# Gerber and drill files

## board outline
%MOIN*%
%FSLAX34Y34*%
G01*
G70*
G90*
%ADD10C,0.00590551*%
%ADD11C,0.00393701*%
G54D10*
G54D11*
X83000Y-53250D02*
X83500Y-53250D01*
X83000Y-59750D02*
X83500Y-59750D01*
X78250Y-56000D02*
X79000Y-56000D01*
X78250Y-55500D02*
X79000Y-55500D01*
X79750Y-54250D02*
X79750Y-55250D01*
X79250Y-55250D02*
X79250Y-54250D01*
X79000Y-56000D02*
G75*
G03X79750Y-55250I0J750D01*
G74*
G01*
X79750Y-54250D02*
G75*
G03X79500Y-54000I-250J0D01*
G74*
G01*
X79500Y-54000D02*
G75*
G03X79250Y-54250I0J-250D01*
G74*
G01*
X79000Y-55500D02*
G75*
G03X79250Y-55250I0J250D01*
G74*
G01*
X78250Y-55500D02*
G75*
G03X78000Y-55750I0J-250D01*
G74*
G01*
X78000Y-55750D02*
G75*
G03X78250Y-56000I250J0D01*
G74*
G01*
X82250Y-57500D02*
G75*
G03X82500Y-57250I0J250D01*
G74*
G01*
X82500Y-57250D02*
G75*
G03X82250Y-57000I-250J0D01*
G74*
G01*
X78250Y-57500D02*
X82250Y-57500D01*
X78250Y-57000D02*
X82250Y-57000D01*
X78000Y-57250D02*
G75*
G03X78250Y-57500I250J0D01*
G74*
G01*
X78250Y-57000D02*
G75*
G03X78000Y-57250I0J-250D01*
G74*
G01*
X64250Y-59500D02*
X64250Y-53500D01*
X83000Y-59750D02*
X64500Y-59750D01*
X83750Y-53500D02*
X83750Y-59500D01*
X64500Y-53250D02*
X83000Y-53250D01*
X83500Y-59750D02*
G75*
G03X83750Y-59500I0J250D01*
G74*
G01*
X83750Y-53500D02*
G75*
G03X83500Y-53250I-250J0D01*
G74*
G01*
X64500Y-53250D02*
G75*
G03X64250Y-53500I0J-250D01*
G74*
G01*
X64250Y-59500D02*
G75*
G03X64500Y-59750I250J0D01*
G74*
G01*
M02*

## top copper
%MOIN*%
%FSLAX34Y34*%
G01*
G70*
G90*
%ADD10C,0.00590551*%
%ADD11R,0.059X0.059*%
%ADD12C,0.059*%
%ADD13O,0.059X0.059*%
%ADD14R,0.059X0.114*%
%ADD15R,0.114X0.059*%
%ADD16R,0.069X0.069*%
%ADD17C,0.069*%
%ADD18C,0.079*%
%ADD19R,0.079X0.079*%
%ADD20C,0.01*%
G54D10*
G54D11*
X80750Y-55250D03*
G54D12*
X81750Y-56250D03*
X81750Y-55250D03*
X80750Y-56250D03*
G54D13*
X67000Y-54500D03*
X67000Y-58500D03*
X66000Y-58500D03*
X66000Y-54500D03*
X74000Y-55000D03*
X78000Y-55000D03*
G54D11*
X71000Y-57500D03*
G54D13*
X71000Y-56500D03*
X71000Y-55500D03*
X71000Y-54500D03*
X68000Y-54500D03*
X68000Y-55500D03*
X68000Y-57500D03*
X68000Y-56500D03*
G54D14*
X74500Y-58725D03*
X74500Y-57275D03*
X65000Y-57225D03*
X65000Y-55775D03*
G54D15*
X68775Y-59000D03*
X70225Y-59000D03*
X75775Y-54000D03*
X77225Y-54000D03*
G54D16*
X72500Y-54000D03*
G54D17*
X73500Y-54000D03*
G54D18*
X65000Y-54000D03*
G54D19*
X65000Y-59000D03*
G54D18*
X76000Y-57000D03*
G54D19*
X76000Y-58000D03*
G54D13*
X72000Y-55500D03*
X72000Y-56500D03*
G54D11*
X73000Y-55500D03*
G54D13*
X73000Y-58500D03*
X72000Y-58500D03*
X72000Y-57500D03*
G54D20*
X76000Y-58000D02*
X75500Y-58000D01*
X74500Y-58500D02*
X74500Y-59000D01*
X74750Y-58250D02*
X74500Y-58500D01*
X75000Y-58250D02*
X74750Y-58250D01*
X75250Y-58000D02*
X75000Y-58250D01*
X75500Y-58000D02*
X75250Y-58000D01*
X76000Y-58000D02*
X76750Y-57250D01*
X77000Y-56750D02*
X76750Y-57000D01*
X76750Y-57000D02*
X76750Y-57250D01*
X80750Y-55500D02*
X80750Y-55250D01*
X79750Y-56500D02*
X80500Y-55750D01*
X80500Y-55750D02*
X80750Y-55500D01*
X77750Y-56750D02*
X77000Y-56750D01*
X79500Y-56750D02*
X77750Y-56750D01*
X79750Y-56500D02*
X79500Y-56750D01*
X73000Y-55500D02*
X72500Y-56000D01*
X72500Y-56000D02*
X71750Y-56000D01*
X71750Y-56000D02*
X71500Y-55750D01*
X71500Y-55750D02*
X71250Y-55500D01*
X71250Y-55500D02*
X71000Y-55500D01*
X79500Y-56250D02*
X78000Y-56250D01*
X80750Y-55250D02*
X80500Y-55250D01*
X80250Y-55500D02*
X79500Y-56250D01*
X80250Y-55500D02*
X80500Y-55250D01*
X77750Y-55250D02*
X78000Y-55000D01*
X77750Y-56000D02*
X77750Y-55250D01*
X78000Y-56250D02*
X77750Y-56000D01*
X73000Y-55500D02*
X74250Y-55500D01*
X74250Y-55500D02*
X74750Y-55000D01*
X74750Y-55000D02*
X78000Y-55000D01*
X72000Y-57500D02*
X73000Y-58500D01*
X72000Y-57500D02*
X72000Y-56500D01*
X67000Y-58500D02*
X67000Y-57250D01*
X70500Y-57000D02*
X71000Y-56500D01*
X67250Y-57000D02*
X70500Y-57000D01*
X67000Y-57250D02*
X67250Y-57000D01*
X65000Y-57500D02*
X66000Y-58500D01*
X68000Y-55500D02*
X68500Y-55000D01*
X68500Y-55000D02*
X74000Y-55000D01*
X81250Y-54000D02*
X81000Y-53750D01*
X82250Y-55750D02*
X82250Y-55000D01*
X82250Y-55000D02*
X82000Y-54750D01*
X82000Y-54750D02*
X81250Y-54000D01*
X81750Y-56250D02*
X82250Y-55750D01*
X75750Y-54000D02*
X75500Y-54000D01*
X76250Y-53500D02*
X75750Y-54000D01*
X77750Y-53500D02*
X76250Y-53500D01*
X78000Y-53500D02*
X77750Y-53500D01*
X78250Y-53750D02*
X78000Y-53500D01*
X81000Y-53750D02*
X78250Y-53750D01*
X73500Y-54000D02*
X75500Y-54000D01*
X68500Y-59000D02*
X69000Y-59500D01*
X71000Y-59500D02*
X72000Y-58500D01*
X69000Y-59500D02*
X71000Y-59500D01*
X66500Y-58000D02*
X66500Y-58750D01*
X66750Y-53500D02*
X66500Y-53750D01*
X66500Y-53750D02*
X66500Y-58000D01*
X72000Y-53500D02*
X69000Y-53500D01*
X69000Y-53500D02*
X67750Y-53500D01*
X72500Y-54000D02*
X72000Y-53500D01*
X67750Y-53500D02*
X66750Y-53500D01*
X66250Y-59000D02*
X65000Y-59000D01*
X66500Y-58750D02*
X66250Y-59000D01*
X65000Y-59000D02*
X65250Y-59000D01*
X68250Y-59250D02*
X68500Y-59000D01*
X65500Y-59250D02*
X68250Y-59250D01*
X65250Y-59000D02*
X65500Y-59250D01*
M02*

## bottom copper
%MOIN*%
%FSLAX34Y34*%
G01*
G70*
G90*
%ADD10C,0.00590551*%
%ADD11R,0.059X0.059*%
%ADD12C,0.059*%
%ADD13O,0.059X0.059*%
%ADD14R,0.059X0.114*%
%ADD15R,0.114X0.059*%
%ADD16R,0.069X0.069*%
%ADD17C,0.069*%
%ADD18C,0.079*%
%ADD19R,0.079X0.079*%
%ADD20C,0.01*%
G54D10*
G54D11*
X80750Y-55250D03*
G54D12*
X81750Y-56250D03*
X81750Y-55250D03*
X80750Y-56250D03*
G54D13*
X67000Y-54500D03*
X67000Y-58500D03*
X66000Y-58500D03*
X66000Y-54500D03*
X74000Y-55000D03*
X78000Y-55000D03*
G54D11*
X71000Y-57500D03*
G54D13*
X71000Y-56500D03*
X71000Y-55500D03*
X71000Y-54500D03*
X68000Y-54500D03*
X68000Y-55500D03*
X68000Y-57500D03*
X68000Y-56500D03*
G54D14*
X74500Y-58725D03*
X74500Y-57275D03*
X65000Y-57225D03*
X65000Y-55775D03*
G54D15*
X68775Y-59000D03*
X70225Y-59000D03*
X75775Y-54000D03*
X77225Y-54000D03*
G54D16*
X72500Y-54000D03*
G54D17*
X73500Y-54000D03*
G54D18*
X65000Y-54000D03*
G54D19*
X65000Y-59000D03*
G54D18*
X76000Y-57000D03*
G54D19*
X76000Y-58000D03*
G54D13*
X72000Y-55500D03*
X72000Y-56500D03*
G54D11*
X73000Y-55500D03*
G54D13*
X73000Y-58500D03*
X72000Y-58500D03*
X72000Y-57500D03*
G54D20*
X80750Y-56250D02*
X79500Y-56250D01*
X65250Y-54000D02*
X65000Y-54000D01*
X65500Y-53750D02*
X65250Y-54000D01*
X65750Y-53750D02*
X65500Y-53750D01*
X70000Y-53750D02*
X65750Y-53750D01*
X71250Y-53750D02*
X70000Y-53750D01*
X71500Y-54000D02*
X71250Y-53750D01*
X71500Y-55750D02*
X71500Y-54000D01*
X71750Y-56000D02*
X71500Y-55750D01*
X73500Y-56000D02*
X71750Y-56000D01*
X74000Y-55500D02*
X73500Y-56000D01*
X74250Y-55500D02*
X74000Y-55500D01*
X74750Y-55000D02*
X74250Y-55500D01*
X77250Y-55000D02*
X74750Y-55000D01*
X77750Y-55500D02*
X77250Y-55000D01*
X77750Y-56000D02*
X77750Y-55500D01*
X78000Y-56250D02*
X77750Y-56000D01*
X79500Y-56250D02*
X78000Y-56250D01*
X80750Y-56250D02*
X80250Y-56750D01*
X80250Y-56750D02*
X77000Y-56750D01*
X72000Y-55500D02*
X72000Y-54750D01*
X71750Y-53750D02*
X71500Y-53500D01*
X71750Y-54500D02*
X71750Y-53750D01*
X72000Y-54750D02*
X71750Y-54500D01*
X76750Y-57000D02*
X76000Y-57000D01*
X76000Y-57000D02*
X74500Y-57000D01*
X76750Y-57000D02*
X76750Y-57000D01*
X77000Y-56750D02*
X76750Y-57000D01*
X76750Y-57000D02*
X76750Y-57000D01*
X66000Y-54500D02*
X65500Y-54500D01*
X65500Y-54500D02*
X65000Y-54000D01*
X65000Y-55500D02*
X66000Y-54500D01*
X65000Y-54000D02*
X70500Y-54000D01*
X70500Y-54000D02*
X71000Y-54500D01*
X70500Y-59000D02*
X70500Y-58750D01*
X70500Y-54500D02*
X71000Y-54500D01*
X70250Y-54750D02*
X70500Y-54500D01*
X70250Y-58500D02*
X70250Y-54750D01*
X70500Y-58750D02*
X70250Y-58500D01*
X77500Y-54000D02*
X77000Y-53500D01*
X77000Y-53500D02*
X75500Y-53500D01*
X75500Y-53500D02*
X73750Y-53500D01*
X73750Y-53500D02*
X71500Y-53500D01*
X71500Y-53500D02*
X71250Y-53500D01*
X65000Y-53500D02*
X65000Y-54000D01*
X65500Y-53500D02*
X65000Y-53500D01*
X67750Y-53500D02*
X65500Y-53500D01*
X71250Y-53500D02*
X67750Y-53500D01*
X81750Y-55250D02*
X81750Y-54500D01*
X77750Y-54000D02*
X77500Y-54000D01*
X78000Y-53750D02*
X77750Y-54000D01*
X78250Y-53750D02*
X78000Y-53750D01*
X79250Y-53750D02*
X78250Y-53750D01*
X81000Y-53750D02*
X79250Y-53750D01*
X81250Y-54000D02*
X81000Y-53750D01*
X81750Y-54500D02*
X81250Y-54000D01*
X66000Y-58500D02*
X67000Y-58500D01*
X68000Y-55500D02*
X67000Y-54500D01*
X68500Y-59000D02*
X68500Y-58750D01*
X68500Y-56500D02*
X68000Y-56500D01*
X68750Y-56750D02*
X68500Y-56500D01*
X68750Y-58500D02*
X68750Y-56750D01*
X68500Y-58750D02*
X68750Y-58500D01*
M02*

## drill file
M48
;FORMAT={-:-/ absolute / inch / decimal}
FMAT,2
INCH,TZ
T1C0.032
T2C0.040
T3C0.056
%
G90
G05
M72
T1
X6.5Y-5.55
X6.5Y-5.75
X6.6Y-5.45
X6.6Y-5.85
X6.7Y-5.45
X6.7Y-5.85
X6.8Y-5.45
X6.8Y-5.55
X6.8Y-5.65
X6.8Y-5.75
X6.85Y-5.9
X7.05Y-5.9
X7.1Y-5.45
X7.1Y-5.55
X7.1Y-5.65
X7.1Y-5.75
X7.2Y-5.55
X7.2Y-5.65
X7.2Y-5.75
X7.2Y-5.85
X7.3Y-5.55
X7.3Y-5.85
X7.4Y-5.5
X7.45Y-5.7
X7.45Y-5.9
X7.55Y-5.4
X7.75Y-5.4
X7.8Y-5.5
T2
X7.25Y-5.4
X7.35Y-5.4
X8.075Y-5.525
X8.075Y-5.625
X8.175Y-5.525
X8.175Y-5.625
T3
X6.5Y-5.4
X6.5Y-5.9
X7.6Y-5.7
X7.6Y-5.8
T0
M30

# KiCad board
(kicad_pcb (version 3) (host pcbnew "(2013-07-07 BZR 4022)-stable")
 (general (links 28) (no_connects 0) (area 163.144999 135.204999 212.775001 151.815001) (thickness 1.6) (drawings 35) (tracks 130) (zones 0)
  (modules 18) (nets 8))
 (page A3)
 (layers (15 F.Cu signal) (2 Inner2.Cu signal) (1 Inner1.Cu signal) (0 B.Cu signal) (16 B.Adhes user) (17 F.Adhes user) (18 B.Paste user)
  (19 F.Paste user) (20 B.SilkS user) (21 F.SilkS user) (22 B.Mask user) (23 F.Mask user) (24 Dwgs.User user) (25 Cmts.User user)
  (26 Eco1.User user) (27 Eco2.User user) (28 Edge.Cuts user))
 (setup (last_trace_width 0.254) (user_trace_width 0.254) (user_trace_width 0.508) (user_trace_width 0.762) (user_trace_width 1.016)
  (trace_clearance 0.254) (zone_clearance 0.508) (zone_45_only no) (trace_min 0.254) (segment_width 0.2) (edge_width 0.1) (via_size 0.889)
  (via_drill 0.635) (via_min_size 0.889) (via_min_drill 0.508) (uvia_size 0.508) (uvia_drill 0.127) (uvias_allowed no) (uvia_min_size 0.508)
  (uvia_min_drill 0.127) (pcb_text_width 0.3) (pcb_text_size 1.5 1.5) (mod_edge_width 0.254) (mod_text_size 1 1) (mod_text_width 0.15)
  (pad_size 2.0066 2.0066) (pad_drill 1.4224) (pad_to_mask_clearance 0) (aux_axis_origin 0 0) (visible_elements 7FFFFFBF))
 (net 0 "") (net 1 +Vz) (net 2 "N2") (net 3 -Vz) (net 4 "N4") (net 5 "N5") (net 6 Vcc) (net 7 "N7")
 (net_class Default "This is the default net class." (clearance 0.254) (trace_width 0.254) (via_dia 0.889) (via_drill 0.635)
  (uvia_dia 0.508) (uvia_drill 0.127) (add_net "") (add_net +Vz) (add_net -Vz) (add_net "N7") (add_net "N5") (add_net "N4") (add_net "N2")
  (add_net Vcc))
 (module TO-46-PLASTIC (layer F.Cu) (at 206.375 141.605)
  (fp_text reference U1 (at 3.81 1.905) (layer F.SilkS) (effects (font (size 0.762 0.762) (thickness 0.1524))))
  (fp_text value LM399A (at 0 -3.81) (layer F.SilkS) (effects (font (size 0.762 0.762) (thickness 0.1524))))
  (pad 1 thru_hole rect (at -1.27 -1.27) (size 1.4986 1.4986) (drill 1.016) (layers *.Cu *.Mask F.SilkS) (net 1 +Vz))
  (pad 3 thru_hole circle (at 1.27 1.27) (size 1.4986 1.4986) (drill 1.016) (layers *.Cu *.Mask F.SilkS) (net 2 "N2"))
  (pad 4 thru_hole circle (at 1.27 -1.27) (size 1.4986 1.4986) (drill 1.016) (layers *.Cu *.Mask F.SilkS) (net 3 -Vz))
  (pad 2 thru_hole circle (at -1.27 1.27) (size 1.4986 1.4986) (drill 1.016) (layers *.Cu *.Mask F.SilkS) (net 3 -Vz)))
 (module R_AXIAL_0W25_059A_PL (layer F.Cu) (at 170.18 138.43 270) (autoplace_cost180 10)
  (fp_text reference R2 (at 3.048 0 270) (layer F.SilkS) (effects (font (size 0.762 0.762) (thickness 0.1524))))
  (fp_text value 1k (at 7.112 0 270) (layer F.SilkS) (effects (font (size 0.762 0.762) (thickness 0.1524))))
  (pad 1 thru_hole oval (at 0 0 270) (size 1.4986 1.4986) (drill 0.8128) (layers *.Cu *.Mask F.SilkS) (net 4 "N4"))
  (pad 2 thru_hole oval (at 10.16 0 270) (size 1.4986 1.4986) (drill 0.8128) (layers *.Cu *.Mask F.SilkS) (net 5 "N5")))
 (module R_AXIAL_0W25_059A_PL (layer F.Cu) (at 167.64 148.59 90) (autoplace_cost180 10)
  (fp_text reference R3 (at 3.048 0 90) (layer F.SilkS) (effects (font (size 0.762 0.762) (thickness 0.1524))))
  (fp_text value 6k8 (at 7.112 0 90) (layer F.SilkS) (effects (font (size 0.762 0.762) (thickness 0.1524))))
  (pad 1 thru_hole oval (at 0 0 90) (size 1.4986 1.4986) (drill 0.8128) (layers *.Cu *.Mask F.SilkS) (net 5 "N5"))
  (pad 2 thru_hole oval (at 10.16 0 90) (size 1.4986 1.4986) (drill 0.8128) (layers *.Cu *.Mask F.SilkS) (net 3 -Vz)))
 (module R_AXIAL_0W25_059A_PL (layer F.Cu) (at 187.96 139.7) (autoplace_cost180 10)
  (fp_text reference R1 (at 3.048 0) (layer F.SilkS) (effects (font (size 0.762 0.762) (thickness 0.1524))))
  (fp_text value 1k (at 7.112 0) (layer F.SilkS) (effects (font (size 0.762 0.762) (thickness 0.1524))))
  (pad 1 thru_hole oval (at 0 0) (size 1.4986 1.4986) (drill 0.8128) (layers *.Cu *.Mask F.SilkS) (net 4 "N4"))
  (pad 2 thru_hole oval (at 10.16 0) (size 1.4986 1.4986) (drill 0.8128) (layers *.Cu *.Mask F.SilkS) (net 1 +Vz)))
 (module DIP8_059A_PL (layer F.Cu) (at 180.34 146.05 90)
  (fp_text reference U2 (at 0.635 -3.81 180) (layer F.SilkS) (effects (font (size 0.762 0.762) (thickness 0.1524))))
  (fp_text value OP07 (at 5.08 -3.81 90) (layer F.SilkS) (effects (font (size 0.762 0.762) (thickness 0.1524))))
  (pad 1 thru_hole rect (at 0 0 90) (size 1.4986 1.4986) (drill 0.8128) (layers *.Cu *.Mask F.SilkS))
  (pad 2 thru_hole oval (at 2.54 0 90) (size 1.4986 1.4986) (drill 0.8128) (layers *.Cu *.Mask F.SilkS) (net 5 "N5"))
  (pad 3 thru_hole oval (at 5.08 0 90) (size 1.4986 1.4986) (drill 0.8128) (layers *.Cu *.Mask F.SilkS) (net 1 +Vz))
  (pad 4 thru_hole oval (at 7.62 0 90) (size 1.4986 1.4986) (drill 0.8128) (layers *.Cu *.Mask F.SilkS) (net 3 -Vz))
  (pad 5 thru_hole oval (at 7.62 -7.62 90) (size 1.4986 1.4986) (drill 0.8128) (layers *.Cu *.Mask F.SilkS))
  (pad 6 thru_hole oval (at 5.08 -7.62 90) (size 1.4986 1.4986) (drill 0.8128) (layers *.Cu *.Mask F.SilkS) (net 4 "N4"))
  (pad 8 thru_hole oval (at 0 -7.62 90) (size 1.4986 1.4986) (drill 0.8128) (layers *.Cu *.Mask F.SilkS))
  (pad 7 thru_hole oval (at 2.54 -7.62 90) (size 1.4986 1.4986) (drill 0.8128) (layers *.Cu *.Mask F.SilkS) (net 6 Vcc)))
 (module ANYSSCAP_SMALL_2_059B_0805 (layer F.Cu) (at 189.23 147.32 90)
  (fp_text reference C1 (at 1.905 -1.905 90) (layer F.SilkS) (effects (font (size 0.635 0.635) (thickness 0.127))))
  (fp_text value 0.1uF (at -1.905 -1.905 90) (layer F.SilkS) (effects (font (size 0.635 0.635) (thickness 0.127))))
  (pad 1 thru_hole rect (at -2.54 0 90) (size 2.8956 1.4986) (drill 0.8128 (offset 0.6985 0)) (layers *.Cu *.Mask F.SilkS) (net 1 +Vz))
  (pad 2 thru_hole rect (at 2.54 0 90) (size 2.8956 1.4986) (drill 0.8128 (offset -0.6985 0)) (layers *.Cu *.Mask F.SilkS) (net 3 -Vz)))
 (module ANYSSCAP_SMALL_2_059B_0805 (layer F.Cu) (at 165.1 143.51 90)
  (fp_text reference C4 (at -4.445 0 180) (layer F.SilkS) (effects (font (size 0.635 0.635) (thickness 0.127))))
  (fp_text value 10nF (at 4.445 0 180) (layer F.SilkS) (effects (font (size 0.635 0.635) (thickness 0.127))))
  (pad 1 thru_hole rect (at -2.54 0 90) (size 2.8956 1.4986) (drill 0.8128 (offset 0.6985 0)) (layers *.Cu *.Mask F.SilkS) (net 5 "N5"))
  (pad 2 thru_hole rect (at 2.54 0 90) (size 2.8956 1.4986) (drill 0.8128 (offset -0.6985 0)) (layers *.Cu *.Mask F.SilkS) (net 3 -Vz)))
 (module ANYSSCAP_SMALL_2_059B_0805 (layer F.Cu) (at 176.53 149.86)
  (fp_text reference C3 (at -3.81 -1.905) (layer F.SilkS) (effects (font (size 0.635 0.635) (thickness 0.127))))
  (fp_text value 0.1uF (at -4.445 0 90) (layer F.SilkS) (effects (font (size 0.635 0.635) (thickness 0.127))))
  (pad 1 thru_hole rect (at -2.54 0) (size 2.8956 1.4986) (drill 0.8128 (offset 0.6985 0)) (layers *.Cu *.Mask F.SilkS) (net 6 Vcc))
  (pad 2 thru_hole rect (at 2.54 0) (size 2.8956 1.4986) (drill 0.8128 (offset -0.6985 0)) (layers *.Cu *.Mask F.SilkS) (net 3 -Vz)))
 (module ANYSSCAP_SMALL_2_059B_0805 (layer F.Cu) (at 194.31 137.16)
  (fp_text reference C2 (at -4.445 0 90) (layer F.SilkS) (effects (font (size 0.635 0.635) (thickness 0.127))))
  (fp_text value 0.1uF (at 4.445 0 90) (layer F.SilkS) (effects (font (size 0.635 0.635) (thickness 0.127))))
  (pad 1 thru_hole rect (at -2.54 0) (size 2.8956 1.4986) (drill 0.8128 (offset 0.6985 0)) (layers *.Cu *.Mask F.SilkS) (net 2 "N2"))
  (pad 2 thru_hole rect (at 2.54 0) (size 2.8956 1.4986) (drill 0.8128 (offset -0.6985 0)) (layers *.Cu *.Mask F.SilkS) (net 3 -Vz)))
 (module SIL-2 (layer F.Cu) (at 184.15 137.16)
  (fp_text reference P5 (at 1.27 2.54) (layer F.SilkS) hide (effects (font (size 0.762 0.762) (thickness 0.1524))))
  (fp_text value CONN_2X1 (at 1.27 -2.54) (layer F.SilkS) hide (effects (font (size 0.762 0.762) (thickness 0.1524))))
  (pad 1 thru_hole rect (at 0 0) (size 1.7526 1.7526) (drill 1.016) (layers *.Cu *.Mask F.SilkS) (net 6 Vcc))
  (pad 2 thru_hole circle (at 2.54 0) (size 1.7526 1.7526) (drill 1.016) (layers *.Cu *.Mask F.SilkS) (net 2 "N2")))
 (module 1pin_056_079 (layer F.Cu) (at 165.1 137.16)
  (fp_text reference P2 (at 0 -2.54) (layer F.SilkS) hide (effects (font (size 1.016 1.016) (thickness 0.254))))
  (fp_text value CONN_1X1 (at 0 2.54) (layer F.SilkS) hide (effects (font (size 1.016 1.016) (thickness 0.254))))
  (pad 1 thru_hole circle (at 0 0) (size 2.0066 2.0066) (drill 1.4224) (layers *.Cu *.Mask F.SilkS) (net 3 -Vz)))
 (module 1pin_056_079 (layer F.Cu) (at 165.1 149.86)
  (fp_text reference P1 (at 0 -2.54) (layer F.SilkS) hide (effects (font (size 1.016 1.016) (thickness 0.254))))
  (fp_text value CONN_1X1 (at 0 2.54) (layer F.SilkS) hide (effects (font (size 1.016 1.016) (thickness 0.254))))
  (pad 1 thru_hole rect (at 0 0) (size 2.0066 2.0066) (drill 1.4224) (layers *.Cu *.Mask F.SilkS) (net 6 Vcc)))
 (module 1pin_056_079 (layer F.Cu) (at 193.04 144.78)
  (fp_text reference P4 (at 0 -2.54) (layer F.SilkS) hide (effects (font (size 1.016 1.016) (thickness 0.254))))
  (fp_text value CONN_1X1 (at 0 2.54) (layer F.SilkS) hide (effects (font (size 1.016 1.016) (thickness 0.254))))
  (pad 1 thru_hole circle (at 0 0) (size 2.0066 2.0066) (drill 1.4224) (layers *.Cu *.Mask F.SilkS) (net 3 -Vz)))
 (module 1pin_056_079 (layer F.Cu) (at 193.04 147.32)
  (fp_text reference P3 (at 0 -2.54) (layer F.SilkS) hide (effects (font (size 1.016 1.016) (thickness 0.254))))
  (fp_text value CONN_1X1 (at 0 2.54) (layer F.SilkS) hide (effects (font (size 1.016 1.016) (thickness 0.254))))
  (pad 1 thru_hole rect (at 0 0) (size 2.0066 2.0066) (drill 1.4224) (layers *.Cu *.Mask F.SilkS) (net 1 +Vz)))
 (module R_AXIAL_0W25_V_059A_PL (layer F.Cu) (at 182.88 140.97 270) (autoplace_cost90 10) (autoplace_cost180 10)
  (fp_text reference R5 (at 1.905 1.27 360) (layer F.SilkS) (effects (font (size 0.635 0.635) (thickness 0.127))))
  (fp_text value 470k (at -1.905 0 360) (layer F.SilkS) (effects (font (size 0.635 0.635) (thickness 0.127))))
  (pad 1 thru_hole oval (at 0 0 270) (size 1.4986 1.4986) (drill 0.8128) (layers *.Cu *.Mask F.SilkS) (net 3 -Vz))
  (pad 2 thru_hole oval (at 2.54 0 270) (size 1.4986 1.4986) (drill 0.8128) (layers *.Cu *.Mask F.SilkS) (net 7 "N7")))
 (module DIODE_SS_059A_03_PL (layer F.Cu) (at 185.42 144.78 90)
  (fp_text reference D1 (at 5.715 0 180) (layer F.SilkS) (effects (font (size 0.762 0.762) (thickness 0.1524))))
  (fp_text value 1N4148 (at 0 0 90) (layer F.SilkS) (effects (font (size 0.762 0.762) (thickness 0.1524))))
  (pad 2 thru_hole rect (at 3.81 0 90) (size 1.4986 1.4986) (drill 0.8128) (layers *.Cu *.Mask F.SilkS) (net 1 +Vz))
  (pad 1 thru_hole oval (at -3.81 0 90) (size 1.4986 1.4986) (drill 0.8128) (layers *.Cu *.Mask F.SilkS) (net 7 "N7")))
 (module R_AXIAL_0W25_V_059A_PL (layer F.Cu) (at 182.88 148.59 90) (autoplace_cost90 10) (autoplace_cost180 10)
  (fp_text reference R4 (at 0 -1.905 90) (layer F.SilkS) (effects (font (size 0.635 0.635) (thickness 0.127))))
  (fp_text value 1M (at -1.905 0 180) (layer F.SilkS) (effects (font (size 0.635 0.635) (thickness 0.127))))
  (pad 1 thru_hole oval (at 0 0 90) (size 1.4986 1.4986) (drill 0.8128) (layers *.Cu *.Mask F.SilkS) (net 6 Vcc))
  (pad 2 thru_hole oval (at 2.54 0 90) (size 1.4986 1.4986) (drill 0.8128) (layers *.Cu *.Mask F.SilkS) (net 7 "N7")))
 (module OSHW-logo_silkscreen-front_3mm (layer F.Cu) (at 196.85 143.51)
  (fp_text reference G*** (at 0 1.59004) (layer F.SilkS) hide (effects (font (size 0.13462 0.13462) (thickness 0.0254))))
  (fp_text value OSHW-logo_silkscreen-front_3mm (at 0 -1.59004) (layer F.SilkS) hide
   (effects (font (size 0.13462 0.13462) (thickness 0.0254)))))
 (gr_line (start 210.82 135.255) (end 212.09 135.255) (angle 90) (layer Edge.Cuts) (width 0.1))
 (gr_line (start 210.82 151.765) (end 212.09 151.765) (angle 90) (layer Edge.Cuts) (width 0.1))
 (gr_line (start 198.755 142.24) (end 200.66 142.24) (angle 90) (layer Edge.Cuts) (width 0.1))
 (gr_line (start 198.755 140.97) (end 200.66 140.97) (angle 90) (layer Edge.Cuts) (width 0.1))
 (gr_line (start 202.565 137.795) (end 202.565 140.335) (angle 90) (layer Edge.Cuts) (width 0.1))
 (gr_line (start 201.295 140.335) (end 201.295 137.795) (angle 90) (layer Edge.Cuts) (width 0.1))
 (gr_arc (start 200.66 140.335) (end 202.565 140.335) (angle 90) (layer Edge.Cuts) (width 0.1))
 (gr_arc (start 201.93 137.795) (end 201.93 137.16) (angle 90) (layer Edge.Cuts) (width 0.1))
 (gr_arc (start 201.93 137.795) (end 201.295 137.795) (angle 90) (layer Edge.Cuts) (width 0.1))
 (gr_arc (start 200.66 140.335) (end 201.295 140.335) (angle 90) (layer Edge.Cuts) (width 0.1))
 (gr_arc (start 198.755 141.605) (end 198.12 141.605) (angle 90) (layer Edge.Cuts) (width 0.1))
 (gr_arc (start 198.755 141.605) (end 198.755 142.24) (angle 90) (layer Edge.Cuts) (width 0.1))
 (gr_arc (start 208.915 145.415) (end 209.55 145.415) (angle 90) (layer Edge.Cuts) (width 0.1))
 (gr_arc (start 208.915 145.415) (end 208.915 144.78) (angle 90) (layer Edge.Cuts) (width 0.1))
 (gr_line (start 198.755 146.05) (end 208.915 146.05) (angle 90) (layer Edge.Cuts) (width 0.1))
 (gr_line (start 198.755 144.78) (end 208.915 144.78) (angle 90) (layer Edge.Cuts) (width 0.1))
 (gr_arc (start 198.755 145.415) (end 198.755 146.05) (angle 90) (layer Edge.Cuts) (width 0.1))
 (gr_arc (start 198.755 145.415) (end 198.12 145.415) (angle 90) (layer Edge.Cuts) (width 0.1))
 (gr_line (start 163.195 151.13) (end 163.195 135.89) (angle 90) (layer Edge.Cuts) (width 0.1))
 (gr_line (start 210.82 151.765) (end 163.83 151.765) (angle 90) (layer Edge.Cuts) (width 0.1))
 (gr_line (start 212.725 135.89) (end 212.725 151.13) (angle 90) (layer Edge.Cuts) (width 0.1))
 (gr_line (start 163.83 135.255) (end 210.82 135.255) (angle 90) (layer Edge.Cuts) (width 0.1))
 (gr_arc (start 212.09 151.13) (end 212.725 151.13) (angle 90) (layer Edge.Cuts) (width 0.1))
 (gr_arc (start 212.09 135.89) (end 212.09 135.255) (angle 90) (layer Edge.Cuts) (width 0.1))
 (gr_arc (start 163.83 135.89) (end 163.195 135.89) (angle 90) (layer Edge.Cuts) (width 0.1))
 (gr_arc (start 163.83 151.13) (end 163.83 151.765) (angle 90) (layer Edge.Cuts) (width 0.1))
 (segment (start 193.04 147.32) (end 191.77 147.32) (width 0.254) (layer F.Cu) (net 1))
 (segment (start 189.23 148.59) (end 189.23 149.86) (width 0.254) (layer F.Cu) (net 1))
 (segment (start 189.865 147.955) (end 189.23 148.59) (width 0.254) (layer F.Cu) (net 1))
 (segment (start 190.5 147.955) (end 189.865 147.955) (width 0.254) (layer F.Cu) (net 1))
 (segment (start 191.135 147.32) (end 190.5 147.955) (width 0.254) (layer F.Cu) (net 1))
 (segment (start 191.77 147.32) (end 191.135 147.32) (width 0.254) (layer F.Cu) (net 1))
 (segment (start 193.04 147.32) (end 194.945 145.415) (width 0.254) (layer F.Cu) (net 1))
 (segment (start 195.58 144.145) (end 194.945 144.78) (width 0.254) (layer F.Cu) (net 1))
 (segment (start 194.945 144.78) (end 194.945 145.415) (width 0.254) (layer F.Cu) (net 1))
 (segment (start 205.105 140.97) (end 205.105 140.335) (width 0.254) (layer F.Cu) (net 1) (status 30))
 (segment (start 202.565 143.51) (end 204.47 141.605) (width 0.254) (layer F.Cu) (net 1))
 (segment (start 204.47 141.605) (end 205.105 140.97) (width 0.254) (layer F.Cu) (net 1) (status 20))
 (segment (start 197.485 144.145) (end 195.58 144.145) (width 0.254) (layer F.Cu) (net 1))
 (segment (start 201.93 144.145) (end 197.485 144.145) (width 0.254) (layer F.Cu) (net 1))
 (segment (start 202.565 143.51) (end 201.93 144.145) (width 0.254) (layer F.Cu) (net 1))
 (segment (start 185.42 140.97) (end 184.15 142.24) (width 0.254) (layer F.Cu) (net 1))
 (segment (start 184.15 142.24) (end 182.245 142.24) (width 0.254) (layer F.Cu) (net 1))
 (segment (start 182.245 142.24) (end 181.61 141.605) (width 0.254) (layer F.Cu) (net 1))
 (segment (start 181.61 141.605) (end 180.975 140.97) (width 0.254) (layer F.Cu) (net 1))
 (segment (start 180.975 140.97) (end 180.34 140.97) (width 0.254) (layer F.Cu) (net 1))
 (segment (start 201.93 142.875) (end 198.12 142.875) (width 0.254) (layer F.Cu) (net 1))
 (segment (start 205.105 140.335) (end 204.47 140.335) (width 0.254) (layer F.Cu) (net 1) (status 30))
 (segment (start 203.835 140.97) (end 201.93 142.875) (width 0.254) (layer F.Cu) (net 1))
 (segment (start 203.835 140.97) (end 204.47 140.335) (width 0.254) (layer F.Cu) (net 1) (status 20))
 (segment (start 197.485 140.335) (end 198.12 139.7) (width 0.254) (layer F.Cu) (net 1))
 (segment (start 197.485 142.24) (end 197.485 140.335) (width 0.254) (layer F.Cu) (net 1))
 (segment (start 198.12 142.875) (end 197.485 142.24) (width 0.254) (layer F.Cu) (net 1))
 (segment (start 185.42 140.97) (end 188.595 140.97) (width 0.254) (layer F.Cu) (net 1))
 (segment (start 188.595 140.97) (end 189.865 139.7) (width 0.254) (layer F.Cu) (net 1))
 (segment (start 189.865 139.7) (end 198.12 139.7) (width 0.254) (layer F.Cu) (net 1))
 (segment (start 205.105 142.875) (end 201.93 142.875) (width 0.254) (layer B.Cu) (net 3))
 (segment (start 165.735 137.16) (end 165.1 137.16) (width 0.254) (layer B.Cu) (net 3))
 (segment (start 166.37 136.525) (end 165.735 137.16) (width 0.254) (layer B.Cu) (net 3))
 (segment (start 167.005 136.525) (end 166.37 136.525) (width 0.254) (layer B.Cu) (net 3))
 (segment (start 177.8 136.525) (end 167.005 136.525) (width 0.254) (layer B.Cu) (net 3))
 (segment (start 180.975 136.525) (end 177.8 136.525) (width 0.254) (layer B.Cu) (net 3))
 (segment (start 181.61 137.16) (end 180.975 136.525) (width 0.254) (layer B.Cu) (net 3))
 (segment (start 181.61 141.605) (end 181.61 137.16) (width 0.254) (layer B.Cu) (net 3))
 (segment (start 182.245 142.24) (end 181.61 141.605) (width 0.254) (layer B.Cu) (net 3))
 (segment (start 186.69 142.24) (end 182.245 142.24) (width 0.254) (layer B.Cu) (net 3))
 (segment (start 187.96 140.97) (end 186.69 142.24) (width 0.254) (layer B.Cu) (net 3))
 (segment (start 188.595 140.97) (end 187.96 140.97) (width 0.254) (layer B.Cu) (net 3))
 (segment (start 189.865 139.7) (end 188.595 140.97) (width 0.254) (layer B.Cu) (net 3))
 (segment (start 196.215 139.7) (end 189.865 139.7) (width 0.254) (layer B.Cu) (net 3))
 (segment (start 197.485 140.97) (end 196.215 139.7) (width 0.254) (layer B.Cu) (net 3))
 (segment (start 197.485 142.24) (end 197.485 140.97) (width 0.254) (layer B.Cu) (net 3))
 (segment (start 198.12 142.875) (end 197.485 142.24) (width 0.254) (layer B.Cu) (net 3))
 (segment (start 201.93 142.875) (end 198.12 142.875) (width 0.254) (layer B.Cu) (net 3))
 (segment (start 205.105 142.875) (end 203.835 144.145) (width 0.254) (layer B.Cu) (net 3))
 (segment (start 203.835 144.145) (end 195.58 144.145) (width 0.254) (layer B.Cu) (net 3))
 (segment (start 182.88 140.97) (end 182.88 139.065) (width 0.254) (layer B.Cu) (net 3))
 (segment (start 182.245 136.525) (end 181.61 135.89) (width 0.254) (layer B.Cu) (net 3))
 (segment (start 182.245 138.43) (end 182.245 136.525) (width 0.254) (layer B.Cu) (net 3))
 (segment (start 182.88 139.065) (end 182.245 138.43) (width 0.254) (layer B.Cu) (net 3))
 (segment (start 194.945 144.78) (end 193.04 144.78) (width 0.254) (layer B.Cu) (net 3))
 (segment (start 193.04 144.78) (end 189.23 144.78) (width 0.254) (layer B.Cu) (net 3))
 (segment (start 194.945 144.78) (end 194.945 144.78) (width 0.254) (layer B.Cu) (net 3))
 (segment (start 195.58 144.145) (end 194.945 144.78) (width 0.254) (layer B.Cu) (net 3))
 (segment (start 194.945 144.78) (end 194.945 144.78) (width 0.254) (layer B.Cu) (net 3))
 (segment (start 167.64 138.43) (end 166.37 138.43) (width 0.254) (layer B.Cu) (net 3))
 (segment (start 166.37 138.43) (end 165.1 137.16) (width 0.254) (layer B.Cu) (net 3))
 (segment (start 165.1 140.97) (end 167.64 138.43) (width 0.254) (layer B.Cu) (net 3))
 (segment (start 165.1 137.16) (end 179.07 137.16) (width 0.254) (layer B.Cu) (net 3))
 (segment (start 179.07 137.16) (end 180.34 138.43) (width 0.254) (layer B.Cu) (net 3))
 (segment (start 179.07 149.86) (end 179.07 149.225) (width 0.254) (layer B.Cu) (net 3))
 (segment (start 179.07 138.43) (end 180.34 138.43) (width 0.254) (layer B.Cu) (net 3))
 (segment (start 178.435 139.065) (end 179.07 138.43) (width 0.254) (layer B.Cu) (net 3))
 (segment (start 178.435 148.59) (end 178.435 139.065) (width 0.254) (layer B.Cu) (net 3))
 (segment (start 179.07 149.225) (end 178.435 148.59) (width 0.254) (layer B.Cu) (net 3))
 (segment (start 196.85 137.16) (end 195.58 135.89) (width 0.254) (layer B.Cu) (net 3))
 (segment (start 195.58 135.89) (end 191.77 135.89) (width 0.254) (layer B.Cu) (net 3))
 (segment (start 191.77 135.89) (end 187.325 135.89) (width 0.254) (layer B.Cu) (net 3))
 (segment (start 187.325 135.89) (end 181.61 135.89) (width 0.254) (layer B.Cu) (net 3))
 (segment (start 181.61 135.89) (end 180.975 135.89) (width 0.254) (layer B.Cu) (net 3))
 (segment (start 165.1 135.89) (end 165.1 137.16) (width 0.254) (layer B.Cu) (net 3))
 (segment (start 166.37 135.89) (end 165.1 135.89) (width 0.254) (layer B.Cu) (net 3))
 (segment (start 172.085 135.89) (end 166.37 135.89) (width 0.254) (layer B.Cu) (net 3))
 (segment (start 180.975 135.89) (end 172.085 135.89) (width 0.254) (layer B.Cu) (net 3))
 (segment (start 207.645 140.335) (end 207.645 138.43) (width 0.254) (layer B.Cu) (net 3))
 (segment (start 197.485 137.16) (end 196.85 137.16) (width 0.254) (layer B.Cu) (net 3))
 (segment (start 198.12 136.525) (end 197.485 137.16) (width 0.254) (layer B.Cu) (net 3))
 (segment (start 198.755 136.525) (end 198.12 136.525) (width 0.254) (layer B.Cu) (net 3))
 (segment (start 201.295 136.525) (end 198.755 136.525) (width 0.254) (layer B.Cu) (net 3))
 (segment (start 205.74 136.525) (end 201.295 136.525) (width 0.254) (layer B.Cu) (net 3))
 (segment (start 206.375 137.16) (end 205.74 136.525) (width 0.254) (layer B.Cu) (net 3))
 (segment (start 207.645 138.43) (end 206.375 137.16) (width 0.254) (layer B.Cu) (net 3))
 (segment (start 182.88 146.05) (end 185.42 148.59) (width 0.254) (layer F.Cu) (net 7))
 (segment (start 182.88 146.05) (end 182.88 143.51) (width 0.254) (layer F.Cu) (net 7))
 (segment (start 170.18 148.59) (end 170.18 145.415) (width 0.254) (layer F.Cu) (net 5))
 (segment (start 179.07 144.78) (end 180.34 143.51) (width 0.254) (layer F.Cu) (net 5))
 (segment (start 170.815 144.78) (end 179.07 144.78) (width 0.254) (layer F.Cu) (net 5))
 (segment (start 170.18 145.415) (end 170.815 144.78) (width 0.254) (layer F.Cu) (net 5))
 (segment (start 167.64 148.59) (end 170.18 148.59) (width 0.254) (layer B.Cu) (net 5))
 (segment (start 165.1 146.05) (end 167.64 148.59) (width 0.254) (layer F.Cu) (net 5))
 (segment (start 172.72 140.97) (end 173.99 139.7) (width 0.254) (layer F.Cu) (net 4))
 (segment (start 173.99 139.7) (end 187.96 139.7) (width 0.254) (layer F.Cu) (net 4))
 (segment (start 172.72 140.97) (end 170.18 138.43) (width 0.254) (layer B.Cu) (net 4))
 (segment (start 206.375 137.16) (end 205.74 136.525) (width 0.254) (layer F.Cu) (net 2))
 (segment (start 208.915 141.605) (end 208.915 139.7) (width 0.254) (layer F.Cu) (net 2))
 (segment (start 208.915 139.7) (end 208.28 139.065) (width 0.254) (layer F.Cu) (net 2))
 (segment (start 208.28 139.065) (end 206.375 137.16) (width 0.254) (layer F.Cu) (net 2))
 (segment (start 207.645 142.875) (end 208.915 141.605) (width 0.254) (layer F.Cu) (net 2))
 (segment (start 192.405 137.16) (end 191.77 137.16) (width 0.254) (layer F.Cu) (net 2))
 (segment (start 193.675 135.89) (end 192.405 137.16) (width 0.254) (layer F.Cu) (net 2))
 (segment (start 197.485 135.89) (end 193.675 135.89) (width 0.254) (layer F.Cu) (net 2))
 (segment (start 198.12 135.89) (end 197.485 135.89) (width 0.254) (layer F.Cu) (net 2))
 (segment (start 198.755 136.525) (end 198.12 135.89) (width 0.254) (layer F.Cu) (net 2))
 (segment (start 205.74 136.525) (end 198.755 136.525) (width 0.254) (layer F.Cu) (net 2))
 (segment (start 186.69 137.16) (end 191.77 137.16) (width 0.254) (layer F.Cu) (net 2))
 (segment (start 173.99 149.86) (end 175.26 151.13) (width 0.254) (layer F.Cu) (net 6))
 (segment (start 180.34 151.13) (end 182.88 148.59) (width 0.254) (layer F.Cu) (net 6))
 (segment (start 175.26 151.13) (end 180.34 151.13) (width 0.254) (layer F.Cu) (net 6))
 (segment (start 168.91 147.32) (end 168.91 149.225) (width 0.254) (layer F.Cu) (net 6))
 (segment (start 169.545 135.89) (end 168.91 136.525) (width 0.254) (layer F.Cu) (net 6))
 (segment (start 168.91 136.525) (end 168.91 147.32) (width 0.254) (layer F.Cu) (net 6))
 (segment (start 182.88 135.89) (end 175.26 135.89) (width 0.254) (layer F.Cu) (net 6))
 (segment (start 175.26 135.89) (end 172.085 135.89) (width 0.254) (layer F.Cu) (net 6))
 (segment (start 184.15 137.16) (end 182.88 135.89) (width 0.254) (layer F.Cu) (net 6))
 (segment (start 172.085 135.89) (end 169.545 135.89) (width 0.254) (layer F.Cu) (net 6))
 (segment (start 168.275 149.86) (end 165.1 149.86) (width 0.254) (layer F.Cu) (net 6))
 (segment (start 168.91 149.225) (end 168.275 149.86) (width 0.254) (layer F.Cu) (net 6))
 (segment (start 173.99 149.86) (end 173.99 149.225) (width 0.254) (layer B.Cu) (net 6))
 (segment (start 173.99 143.51) (end 172.72 143.51) (width 0.254) (layer B.Cu) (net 6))
 (segment (start 174.625 144.145) (end 173.99 143.51) (width 0.254) (layer B.Cu) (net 6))
 (segment (start 174.625 148.59) (end 174.625 144.145) (width 0.254) (layer B.Cu) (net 6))
 (segment (start 173.99 149.225) (end 174.625 148.59) (width 0.254) (layer B.Cu) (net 6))
 (segment (start 165.1 149.86) (end 165.735 149.86) (width 0.254) (layer F.Cu) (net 6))
 (segment (start 173.355 150.495) (end 173.99 149.86) (width 0.254) (layer F.Cu) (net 6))
 (segment (start 166.37 150.495) (end 173.355 150.495) (width 0.254) (layer F.Cu) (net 6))
 (segment (start 165.735 149.86) (end 166.37 150.495) (width 0.254) (layer F.Cu) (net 6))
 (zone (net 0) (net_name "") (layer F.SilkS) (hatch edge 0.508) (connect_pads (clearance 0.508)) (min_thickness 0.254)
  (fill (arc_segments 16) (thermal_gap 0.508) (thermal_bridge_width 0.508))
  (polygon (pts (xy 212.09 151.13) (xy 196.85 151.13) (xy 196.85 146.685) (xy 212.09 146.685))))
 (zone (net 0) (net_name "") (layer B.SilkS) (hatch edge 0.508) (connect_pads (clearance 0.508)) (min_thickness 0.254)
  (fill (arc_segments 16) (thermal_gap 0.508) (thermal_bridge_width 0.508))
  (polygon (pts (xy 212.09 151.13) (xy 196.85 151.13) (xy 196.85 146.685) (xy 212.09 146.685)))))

